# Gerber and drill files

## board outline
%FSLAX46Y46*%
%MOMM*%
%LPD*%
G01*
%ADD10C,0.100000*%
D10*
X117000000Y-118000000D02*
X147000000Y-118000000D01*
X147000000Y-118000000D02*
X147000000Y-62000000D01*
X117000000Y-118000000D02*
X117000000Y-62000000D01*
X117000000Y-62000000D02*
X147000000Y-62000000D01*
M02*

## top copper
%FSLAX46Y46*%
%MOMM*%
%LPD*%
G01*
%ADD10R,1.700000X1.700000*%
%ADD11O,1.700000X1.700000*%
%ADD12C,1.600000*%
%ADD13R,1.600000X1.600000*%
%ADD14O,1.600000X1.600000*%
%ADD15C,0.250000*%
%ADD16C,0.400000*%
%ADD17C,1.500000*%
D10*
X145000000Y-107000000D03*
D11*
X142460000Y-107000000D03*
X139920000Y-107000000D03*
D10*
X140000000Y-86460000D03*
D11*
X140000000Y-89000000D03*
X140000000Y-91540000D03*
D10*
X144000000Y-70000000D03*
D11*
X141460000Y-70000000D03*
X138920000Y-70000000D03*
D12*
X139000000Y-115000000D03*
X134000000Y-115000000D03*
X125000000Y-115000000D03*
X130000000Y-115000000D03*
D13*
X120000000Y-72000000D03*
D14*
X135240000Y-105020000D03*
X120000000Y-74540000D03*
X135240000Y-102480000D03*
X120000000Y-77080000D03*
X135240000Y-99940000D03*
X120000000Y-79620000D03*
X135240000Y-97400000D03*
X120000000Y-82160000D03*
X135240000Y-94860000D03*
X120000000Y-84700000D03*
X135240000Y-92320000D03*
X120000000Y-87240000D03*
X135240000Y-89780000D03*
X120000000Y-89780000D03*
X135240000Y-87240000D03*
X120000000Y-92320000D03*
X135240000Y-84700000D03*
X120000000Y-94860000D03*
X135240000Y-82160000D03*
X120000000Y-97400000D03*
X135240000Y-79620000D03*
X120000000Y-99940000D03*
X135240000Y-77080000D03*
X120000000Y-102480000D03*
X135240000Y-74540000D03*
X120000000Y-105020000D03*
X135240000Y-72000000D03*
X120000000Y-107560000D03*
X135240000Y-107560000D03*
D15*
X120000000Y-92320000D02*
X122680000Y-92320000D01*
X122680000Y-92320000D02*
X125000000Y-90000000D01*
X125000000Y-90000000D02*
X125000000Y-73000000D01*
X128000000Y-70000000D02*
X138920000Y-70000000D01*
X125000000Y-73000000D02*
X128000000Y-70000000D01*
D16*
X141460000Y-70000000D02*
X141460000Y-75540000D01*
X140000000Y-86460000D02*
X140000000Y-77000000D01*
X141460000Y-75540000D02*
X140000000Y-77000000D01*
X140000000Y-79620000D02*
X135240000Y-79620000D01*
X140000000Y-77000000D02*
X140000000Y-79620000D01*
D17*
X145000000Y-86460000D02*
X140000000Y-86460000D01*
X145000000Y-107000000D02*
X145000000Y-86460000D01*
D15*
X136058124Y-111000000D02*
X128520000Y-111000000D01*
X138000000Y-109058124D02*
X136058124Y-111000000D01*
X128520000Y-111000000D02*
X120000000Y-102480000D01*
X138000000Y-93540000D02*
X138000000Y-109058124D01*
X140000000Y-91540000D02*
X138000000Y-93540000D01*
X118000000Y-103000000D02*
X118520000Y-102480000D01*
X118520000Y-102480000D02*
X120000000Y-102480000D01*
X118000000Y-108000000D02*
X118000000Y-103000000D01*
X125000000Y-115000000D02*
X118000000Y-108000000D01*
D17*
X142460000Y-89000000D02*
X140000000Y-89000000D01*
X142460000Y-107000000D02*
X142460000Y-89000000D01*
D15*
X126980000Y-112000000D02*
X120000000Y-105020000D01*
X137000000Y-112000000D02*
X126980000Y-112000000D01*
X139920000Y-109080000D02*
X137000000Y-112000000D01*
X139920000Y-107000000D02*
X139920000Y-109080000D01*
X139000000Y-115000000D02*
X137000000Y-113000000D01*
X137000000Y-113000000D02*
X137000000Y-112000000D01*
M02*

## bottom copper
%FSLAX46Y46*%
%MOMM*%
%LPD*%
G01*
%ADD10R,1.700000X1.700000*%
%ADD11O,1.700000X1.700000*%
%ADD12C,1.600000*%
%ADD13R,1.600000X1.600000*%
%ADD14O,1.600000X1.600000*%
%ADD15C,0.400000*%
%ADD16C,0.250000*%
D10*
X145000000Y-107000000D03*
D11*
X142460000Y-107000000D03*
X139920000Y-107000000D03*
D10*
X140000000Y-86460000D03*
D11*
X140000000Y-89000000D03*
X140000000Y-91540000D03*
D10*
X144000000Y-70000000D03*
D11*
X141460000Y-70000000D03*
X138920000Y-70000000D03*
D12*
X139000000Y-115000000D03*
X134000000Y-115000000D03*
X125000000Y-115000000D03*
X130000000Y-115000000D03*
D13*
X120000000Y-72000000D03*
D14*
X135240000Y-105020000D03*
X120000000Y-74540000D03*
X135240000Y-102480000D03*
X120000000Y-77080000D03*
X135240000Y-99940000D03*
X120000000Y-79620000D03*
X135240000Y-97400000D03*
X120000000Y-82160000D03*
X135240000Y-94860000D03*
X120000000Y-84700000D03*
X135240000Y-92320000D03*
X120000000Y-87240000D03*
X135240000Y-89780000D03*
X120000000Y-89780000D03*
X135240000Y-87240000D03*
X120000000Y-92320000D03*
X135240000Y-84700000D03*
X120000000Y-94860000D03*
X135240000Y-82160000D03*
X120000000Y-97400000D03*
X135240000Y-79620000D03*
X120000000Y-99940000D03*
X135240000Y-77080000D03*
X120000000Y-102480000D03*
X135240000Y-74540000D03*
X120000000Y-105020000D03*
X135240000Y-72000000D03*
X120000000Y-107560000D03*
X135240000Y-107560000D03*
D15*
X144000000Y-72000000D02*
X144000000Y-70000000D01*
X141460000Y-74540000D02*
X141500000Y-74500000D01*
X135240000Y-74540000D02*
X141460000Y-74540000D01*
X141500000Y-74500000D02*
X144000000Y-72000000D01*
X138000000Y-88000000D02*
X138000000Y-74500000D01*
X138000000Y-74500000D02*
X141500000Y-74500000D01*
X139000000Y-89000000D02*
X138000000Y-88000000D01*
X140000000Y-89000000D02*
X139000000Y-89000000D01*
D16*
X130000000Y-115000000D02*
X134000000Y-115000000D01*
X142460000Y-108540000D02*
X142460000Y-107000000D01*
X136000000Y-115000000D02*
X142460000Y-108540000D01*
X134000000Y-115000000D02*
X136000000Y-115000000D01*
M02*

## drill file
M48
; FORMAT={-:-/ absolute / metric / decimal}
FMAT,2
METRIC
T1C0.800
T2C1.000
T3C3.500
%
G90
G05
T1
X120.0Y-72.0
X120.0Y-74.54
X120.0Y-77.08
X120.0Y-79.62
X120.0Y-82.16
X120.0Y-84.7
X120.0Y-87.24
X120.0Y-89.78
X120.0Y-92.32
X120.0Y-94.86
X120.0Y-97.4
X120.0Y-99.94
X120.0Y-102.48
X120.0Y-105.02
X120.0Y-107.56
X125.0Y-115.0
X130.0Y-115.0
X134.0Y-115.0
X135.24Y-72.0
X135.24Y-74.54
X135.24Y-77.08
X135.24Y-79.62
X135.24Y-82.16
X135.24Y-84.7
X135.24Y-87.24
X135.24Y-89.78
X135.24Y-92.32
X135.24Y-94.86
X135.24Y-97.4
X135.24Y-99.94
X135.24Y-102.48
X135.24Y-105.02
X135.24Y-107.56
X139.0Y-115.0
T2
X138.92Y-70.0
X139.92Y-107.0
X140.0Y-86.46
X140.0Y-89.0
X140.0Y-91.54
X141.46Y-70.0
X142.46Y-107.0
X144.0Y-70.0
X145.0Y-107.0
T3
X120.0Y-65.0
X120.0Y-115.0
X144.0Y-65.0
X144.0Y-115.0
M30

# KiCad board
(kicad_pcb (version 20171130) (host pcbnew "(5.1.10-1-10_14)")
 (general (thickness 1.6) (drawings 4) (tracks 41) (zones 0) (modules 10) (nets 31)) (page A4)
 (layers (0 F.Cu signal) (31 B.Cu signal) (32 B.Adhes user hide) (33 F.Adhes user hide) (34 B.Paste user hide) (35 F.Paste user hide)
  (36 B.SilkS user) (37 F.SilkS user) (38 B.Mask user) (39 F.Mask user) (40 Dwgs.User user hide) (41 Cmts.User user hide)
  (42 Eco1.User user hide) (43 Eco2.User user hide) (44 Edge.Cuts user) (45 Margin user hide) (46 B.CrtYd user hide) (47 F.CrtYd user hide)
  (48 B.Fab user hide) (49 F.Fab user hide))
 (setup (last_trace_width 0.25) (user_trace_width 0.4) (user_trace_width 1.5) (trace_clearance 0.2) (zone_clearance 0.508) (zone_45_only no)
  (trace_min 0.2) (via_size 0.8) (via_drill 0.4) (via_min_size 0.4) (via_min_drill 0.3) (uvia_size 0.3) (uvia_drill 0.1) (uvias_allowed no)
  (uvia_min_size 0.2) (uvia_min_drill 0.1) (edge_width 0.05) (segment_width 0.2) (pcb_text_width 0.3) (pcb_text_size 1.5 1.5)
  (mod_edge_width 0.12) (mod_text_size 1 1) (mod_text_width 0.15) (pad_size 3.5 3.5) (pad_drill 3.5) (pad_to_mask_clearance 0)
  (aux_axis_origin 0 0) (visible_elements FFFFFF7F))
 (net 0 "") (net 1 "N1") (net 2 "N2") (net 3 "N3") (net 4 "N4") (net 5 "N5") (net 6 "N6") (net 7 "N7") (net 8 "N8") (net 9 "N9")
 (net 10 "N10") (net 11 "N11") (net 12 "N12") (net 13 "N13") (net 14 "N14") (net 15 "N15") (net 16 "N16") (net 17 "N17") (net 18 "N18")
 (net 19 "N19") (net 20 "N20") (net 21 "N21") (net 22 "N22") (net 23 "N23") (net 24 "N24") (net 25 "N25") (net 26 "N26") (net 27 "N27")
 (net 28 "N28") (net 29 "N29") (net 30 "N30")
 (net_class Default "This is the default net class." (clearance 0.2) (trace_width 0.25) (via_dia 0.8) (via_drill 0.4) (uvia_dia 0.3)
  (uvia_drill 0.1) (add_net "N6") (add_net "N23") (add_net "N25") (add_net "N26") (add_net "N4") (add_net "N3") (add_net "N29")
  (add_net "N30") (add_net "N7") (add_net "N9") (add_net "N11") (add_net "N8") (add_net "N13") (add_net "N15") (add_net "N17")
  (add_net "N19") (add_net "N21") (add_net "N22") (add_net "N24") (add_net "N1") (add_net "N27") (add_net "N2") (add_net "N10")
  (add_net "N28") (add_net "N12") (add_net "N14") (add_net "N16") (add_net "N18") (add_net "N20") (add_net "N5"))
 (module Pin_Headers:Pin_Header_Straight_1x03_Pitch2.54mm (layer F.Cu) (at 145 107 270)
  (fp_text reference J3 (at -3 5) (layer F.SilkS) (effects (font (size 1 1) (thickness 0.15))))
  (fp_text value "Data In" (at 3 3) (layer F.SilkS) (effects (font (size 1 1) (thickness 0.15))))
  (pad 1 thru_hole rect (at 0 0 270) (size 1.7 1.7) (drill 1) (layers *.Cu *.Mask) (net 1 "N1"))
  (pad 2 thru_hole oval (at 0 2.54 270) (size 1.7 1.7) (drill 1) (layers *.Cu *.Mask) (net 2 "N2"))
  (pad 3 thru_hole oval (at 0 5.08 270) (size 1.7 1.7) (drill 1) (layers *.Cu *.Mask) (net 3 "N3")))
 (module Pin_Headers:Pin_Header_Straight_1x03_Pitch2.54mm (layer F.Cu) (at 140 86.46)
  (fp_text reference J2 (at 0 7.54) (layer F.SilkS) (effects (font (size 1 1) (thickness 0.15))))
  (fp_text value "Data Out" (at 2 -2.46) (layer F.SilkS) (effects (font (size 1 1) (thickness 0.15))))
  (pad 1 thru_hole rect (at 0 0) (size 1.7 1.7) (drill 1) (layers *.Cu *.Mask) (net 1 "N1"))
  (pad 2 thru_hole oval (at 0 2.54) (size 1.7 1.7) (drill 1) (layers *.Cu *.Mask) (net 2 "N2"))
  (pad 3 thru_hole oval (at 0 5.08) (size 1.7 1.7) (drill 1) (layers *.Cu *.Mask) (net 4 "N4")))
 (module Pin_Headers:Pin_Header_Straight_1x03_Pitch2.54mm (layer F.Cu) (at 144 70 270)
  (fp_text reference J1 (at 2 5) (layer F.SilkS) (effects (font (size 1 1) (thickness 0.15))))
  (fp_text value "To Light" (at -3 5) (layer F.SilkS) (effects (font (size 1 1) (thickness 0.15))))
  (pad 1 thru_hole rect (at 0 0 270) (size 1.7 1.7) (drill 1) (layers *.Cu *.Mask) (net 2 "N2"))
  (pad 2 thru_hole oval (at 0 2.54 270) (size 1.7 1.7) (drill 1) (layers *.Cu *.Mask) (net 1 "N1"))
  (pad 3 thru_hole oval (at 0 5.08 270) (size 1.7 1.7) (drill 1) (layers *.Cu *.Mask) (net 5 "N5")))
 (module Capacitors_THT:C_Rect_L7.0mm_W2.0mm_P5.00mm (layer F.Cu) (at 139 115 180)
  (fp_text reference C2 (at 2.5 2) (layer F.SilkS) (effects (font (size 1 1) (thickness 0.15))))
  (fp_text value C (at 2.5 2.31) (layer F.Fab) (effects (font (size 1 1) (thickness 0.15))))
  (pad 1 thru_hole circle (at 0 0 180) (size 1.6 1.6) (drill 0.8) (layers *.Cu *.Mask) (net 3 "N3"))
  (pad 2 thru_hole circle (at 5 0 180) (size 1.6 1.6) (drill 0.8) (layers *.Cu *.Mask) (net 2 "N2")))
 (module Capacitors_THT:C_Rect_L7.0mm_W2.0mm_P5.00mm (layer F.Cu) (at 125 115)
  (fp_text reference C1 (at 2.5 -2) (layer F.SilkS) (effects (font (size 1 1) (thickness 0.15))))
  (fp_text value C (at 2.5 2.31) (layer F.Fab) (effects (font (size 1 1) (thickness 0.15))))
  (pad 1 thru_hole circle (at 0 0) (size 1.6 1.6) (drill 0.8) (layers *.Cu *.Mask) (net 4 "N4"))
  (pad 2 thru_hole circle (at 5 0) (size 1.6 1.6) (drill 0.8) (layers *.Cu *.Mask) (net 2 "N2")))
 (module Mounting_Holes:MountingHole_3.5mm (layer F.Cu) (at 144 65)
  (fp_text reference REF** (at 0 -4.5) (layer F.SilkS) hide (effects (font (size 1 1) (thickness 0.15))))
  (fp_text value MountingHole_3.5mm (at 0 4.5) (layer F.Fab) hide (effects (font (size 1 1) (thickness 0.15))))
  (pad "" np_thru_hole circle (at 0 0) (size 3.5 3.5) (drill 3.5) (layers *.Cu *.Mask)))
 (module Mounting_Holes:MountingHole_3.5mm (layer F.Cu) (at 144 115)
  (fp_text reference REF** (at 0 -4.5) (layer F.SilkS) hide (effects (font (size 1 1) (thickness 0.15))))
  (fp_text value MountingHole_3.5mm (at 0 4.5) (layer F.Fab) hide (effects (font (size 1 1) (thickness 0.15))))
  (pad "" np_thru_hole circle (at 0 0) (size 3.5 3.5) (drill 3.5) (layers *.Cu *.Mask)))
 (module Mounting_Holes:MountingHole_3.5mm (layer F.Cu) (at 120 115)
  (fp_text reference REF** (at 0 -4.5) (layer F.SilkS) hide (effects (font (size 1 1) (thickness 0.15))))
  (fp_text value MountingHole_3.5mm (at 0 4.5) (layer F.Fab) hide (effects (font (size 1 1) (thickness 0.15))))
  (pad "" np_thru_hole circle (at 0 0) (size 3.5 3.5) (drill 3.5) (layers *.Cu *.Mask)))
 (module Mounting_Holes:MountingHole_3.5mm (layer F.Cu) (at 120 65)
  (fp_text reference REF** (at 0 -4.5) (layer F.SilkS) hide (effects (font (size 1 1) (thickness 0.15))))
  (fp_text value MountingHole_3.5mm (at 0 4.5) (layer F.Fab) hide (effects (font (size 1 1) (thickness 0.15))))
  (pad "" np_thru_hole circle (at 0 0) (size 3.5 3.5) (drill 3.5) (layers *.Cu *.Mask)))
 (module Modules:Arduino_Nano (layer F.Cu) (at 120 72)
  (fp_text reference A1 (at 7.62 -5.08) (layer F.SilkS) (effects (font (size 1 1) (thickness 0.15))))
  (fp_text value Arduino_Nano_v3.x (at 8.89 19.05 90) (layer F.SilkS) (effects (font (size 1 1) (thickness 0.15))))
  (pad 1 thru_hole rect (at 0 0) (size 1.6 1.6) (drill 0.8) (layers *.Cu *.Mask) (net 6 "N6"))
  (pad 17 thru_hole oval (at 15.24 33.02) (size 1.6 1.6) (drill 0.8) (layers *.Cu *.Mask) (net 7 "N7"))
  (pad 2 thru_hole oval (at 0 2.54) (size 1.6 1.6) (drill 0.8) (layers *.Cu *.Mask) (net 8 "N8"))
  (pad 18 thru_hole oval (at 15.24 30.48) (size 1.6 1.6) (drill 0.8) (layers *.Cu *.Mask) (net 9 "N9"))
  (pad 3 thru_hole oval (at 0 5.08) (size 1.6 1.6) (drill 0.8) (layers *.Cu *.Mask) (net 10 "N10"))
  (pad 19 thru_hole oval (at 15.24 27.94) (size 1.6 1.6) (drill 0.8) (layers *.Cu *.Mask) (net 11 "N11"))
  (pad 4 thru_hole oval (at 0 7.62) (size 1.6 1.6) (drill 0.8) (layers *.Cu *.Mask) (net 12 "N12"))
  (pad 20 thru_hole oval (at 15.24 25.4) (size 1.6 1.6) (drill 0.8) (layers *.Cu *.Mask) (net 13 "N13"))
  (pad 5 thru_hole oval (at 0 10.16) (size 1.6 1.6) (drill 0.8) (layers *.Cu *.Mask) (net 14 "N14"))
  (pad 21 thru_hole oval (at 15.24 22.86) (size 1.6 1.6) (drill 0.8) (layers *.Cu *.Mask) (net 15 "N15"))
  (pad 6 thru_hole oval (at 0 12.7) (size 1.6 1.6) (drill 0.8) (layers *.Cu *.Mask) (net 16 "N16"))
  (pad 22 thru_hole oval (at 15.24 20.32) (size 1.6 1.6) (drill 0.8) (layers *.Cu *.Mask) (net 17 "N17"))
  (pad 7 thru_hole oval (at 0 15.24) (size 1.6 1.6) (drill 0.8) (layers *.Cu *.Mask) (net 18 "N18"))
  (pad 23 thru_hole oval (at 15.24 17.78) (size 1.6 1.6) (drill 0.8) (layers *.Cu *.Mask) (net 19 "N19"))
  (pad 8 thru_hole oval (at 0 17.78) (size 1.6 1.6) (drill 0.8) (layers *.Cu *.Mask) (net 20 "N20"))
  (pad 24 thru_hole oval (at 15.24 15.24) (size 1.6 1.6) (drill 0.8) (layers *.Cu *.Mask) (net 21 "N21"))
  (pad 9 thru_hole oval (at 0 20.32) (size 1.6 1.6) (drill 0.8) (layers *.Cu *.Mask) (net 5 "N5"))
  (pad 25 thru_hole oval (at 15.24 12.7) (size 1.6 1.6) (drill 0.8) (layers *.Cu *.Mask) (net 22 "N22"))
  (pad 10 thru_hole oval (at 0 22.86) (size 1.6 1.6) (drill 0.8) (layers *.Cu *.Mask) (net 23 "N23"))
  (pad 26 thru_hole oval (at 15.24 10.16) (size 1.6 1.6) (drill 0.8) (layers *.Cu *.Mask) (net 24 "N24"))
  (pad 11 thru_hole oval (at 0 25.4) (size 1.6 1.6) (drill 0.8) (layers *.Cu *.Mask) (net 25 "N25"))
  (pad 27 thru_hole oval (at 15.24 7.62) (size 1.6 1.6) (drill 0.8) (layers *.Cu *.Mask) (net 1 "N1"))
  (pad 12 thru_hole oval (at 0 27.94) (size 1.6 1.6) (drill 0.8) (layers *.Cu *.Mask) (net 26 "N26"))
  (pad 28 thru_hole oval (at 15.24 5.08) (size 1.6 1.6) (drill 0.8) (layers *.Cu *.Mask) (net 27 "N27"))
  (pad 13 thru_hole oval (at 0 30.48) (size 1.6 1.6) (drill 0.8) (layers *.Cu *.Mask) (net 4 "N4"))
  (pad 29 thru_hole oval (at 15.24 2.54) (size 1.6 1.6) (drill 0.8) (layers *.Cu *.Mask) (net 2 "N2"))
  (pad 14 thru_hole oval (at 0 33.02) (size 1.6 1.6) (drill 0.8) (layers *.Cu *.Mask) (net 3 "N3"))
  (pad 30 thru_hole oval (at 15.24 0) (size 1.6 1.6) (drill 0.8) (layers *.Cu *.Mask) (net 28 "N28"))
  (pad 15 thru_hole oval (at 0 35.56) (size 1.6 1.6) (drill 0.8) (layers *.Cu *.Mask) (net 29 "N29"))
  (pad 16 thru_hole oval (at 15.24 35.56) (size 1.6 1.6) (drill 0.8) (layers *.Cu *.Mask) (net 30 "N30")))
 (gr_line (start 117 118) (end 147 118) (layer Edge.Cuts) (width 0.1))
 (gr_line (start 147 118) (end 147 62) (layer Edge.Cuts) (width 0.1))
 (gr_line (start 117 118) (end 117 62) (layer Edge.Cuts) (width 0.1))
 (gr_line (start 117 62) (end 147 62) (layer Edge.Cuts) (width 0.1))
 (segment (start 120 92.32) (end 122.68 92.32) (width 0.25) (layer F.Cu) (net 5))
 (segment (start 122.68 92.32) (end 125 90) (width 0.25) (layer F.Cu) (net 5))
 (segment (start 125 90) (end 125 73) (width 0.25) (layer F.Cu) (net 5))
 (segment (start 128 70) (end 138.92 70) (width 0.25) (layer F.Cu) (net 5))
 (segment (start 125 73) (end 128 70) (width 0.25) (layer F.Cu) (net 5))
 (segment (start 141.46 70) (end 141.46 75.54) (width 0.4) (layer F.Cu) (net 1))
 (segment (start 140 86.46) (end 140 77) (width 0.4) (layer F.Cu) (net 1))
 (segment (start 141.46 75.54) (end 140 77) (width 0.4) (layer F.Cu) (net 1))
 (segment (start 140 79.62) (end 135.24 79.62) (width 0.4) (layer F.Cu) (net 1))
 (segment (start 140 77) (end 140 79.62) (width 0.4) (layer F.Cu) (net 1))
 (segment (start 145 86.46) (end 140 86.46) (width 1.5) (layer F.Cu) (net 1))
 (segment (start 145 107) (end 145 86.46) (width 1.5) (layer F.Cu) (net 1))
 (segment (start 136.058124 111) (end 128.52 111) (width 0.25) (layer F.Cu) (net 4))
 (segment (start 138 109.058124) (end 136.058124 111) (width 0.25) (layer F.Cu) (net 4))
 (segment (start 128.52 111) (end 120 102.48) (width 0.25) (layer F.Cu) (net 4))
 (segment (start 138 93.54) (end 138 109.058124) (width 0.25) (layer F.Cu) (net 4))
 (segment (start 140 91.54) (end 138 93.54) (width 0.25) (layer F.Cu) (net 4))
 (segment (start 118 103) (end 118.52 102.48) (width 0.25) (layer F.Cu) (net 4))
 (segment (start 118.52 102.48) (end 120 102.48) (width 0.25) (layer F.Cu) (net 4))
 (segment (start 118 108) (end 118 103) (width 0.25) (layer F.Cu) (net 4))
 (segment (start 125 115) (end 118 108) (width 0.25) (layer F.Cu) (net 4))
 (segment (start 142.46 89) (end 140 89) (width 1.5) (layer F.Cu) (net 2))
 (segment (start 142.46 107) (end 142.46 89) (width 1.5) (layer F.Cu) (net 2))
 (segment (start 144 72) (end 144 70) (width 0.4) (layer B.Cu) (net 2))
 (segment (start 141.46 74.54) (end 141.5 74.5) (width 0.4) (layer B.Cu) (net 2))
 (segment (start 135.24 74.54) (end 141.46 74.54) (width 0.4) (layer B.Cu) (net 2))
 (segment (start 141.5 74.5) (end 144 72) (width 0.4) (layer B.Cu) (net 2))
 (segment (start 138 88) (end 138 74.5) (width 0.4) (layer B.Cu) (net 2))
 (segment (start 138 74.5) (end 141.5 74.5) (width 0.4) (layer B.Cu) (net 2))
 (segment (start 139 89) (end 138 88) (width 0.4) (layer B.Cu) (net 2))
 (segment (start 140 89) (end 139 89) (width 0.4) (layer B.Cu) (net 2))
 (segment (start 130 115) (end 134 115) (width 0.25) (layer B.Cu) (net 2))
 (segment (start 142.46 108.54) (end 142.46 107) (width 0.25) (layer B.Cu) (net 2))
 (segment (start 136 115) (end 142.46 108.54) (width 0.25) (layer B.Cu) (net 2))
 (segment (start 134 115) (end 136 115) (width 0.25) (layer B.Cu) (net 2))
 (segment (start 126.98 112) (end 120 105.02) (width 0.25) (layer F.Cu) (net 3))
 (segment (start 137 112) (end 126.98 112) (width 0.25) (layer F.Cu) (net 3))
 (segment (start 139.92 109.08) (end 137 112) (width 0.25) (layer F.Cu) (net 3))
 (segment (start 139.92 107) (end 139.92 109.08) (width 0.25) (layer F.Cu) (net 3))
 (segment (start 139 115) (end 137 113) (width 0.25) (layer F.Cu) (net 3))
 (segment (start 137 113) (end 137 112) (width 0.25) (layer F.Cu) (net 3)))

